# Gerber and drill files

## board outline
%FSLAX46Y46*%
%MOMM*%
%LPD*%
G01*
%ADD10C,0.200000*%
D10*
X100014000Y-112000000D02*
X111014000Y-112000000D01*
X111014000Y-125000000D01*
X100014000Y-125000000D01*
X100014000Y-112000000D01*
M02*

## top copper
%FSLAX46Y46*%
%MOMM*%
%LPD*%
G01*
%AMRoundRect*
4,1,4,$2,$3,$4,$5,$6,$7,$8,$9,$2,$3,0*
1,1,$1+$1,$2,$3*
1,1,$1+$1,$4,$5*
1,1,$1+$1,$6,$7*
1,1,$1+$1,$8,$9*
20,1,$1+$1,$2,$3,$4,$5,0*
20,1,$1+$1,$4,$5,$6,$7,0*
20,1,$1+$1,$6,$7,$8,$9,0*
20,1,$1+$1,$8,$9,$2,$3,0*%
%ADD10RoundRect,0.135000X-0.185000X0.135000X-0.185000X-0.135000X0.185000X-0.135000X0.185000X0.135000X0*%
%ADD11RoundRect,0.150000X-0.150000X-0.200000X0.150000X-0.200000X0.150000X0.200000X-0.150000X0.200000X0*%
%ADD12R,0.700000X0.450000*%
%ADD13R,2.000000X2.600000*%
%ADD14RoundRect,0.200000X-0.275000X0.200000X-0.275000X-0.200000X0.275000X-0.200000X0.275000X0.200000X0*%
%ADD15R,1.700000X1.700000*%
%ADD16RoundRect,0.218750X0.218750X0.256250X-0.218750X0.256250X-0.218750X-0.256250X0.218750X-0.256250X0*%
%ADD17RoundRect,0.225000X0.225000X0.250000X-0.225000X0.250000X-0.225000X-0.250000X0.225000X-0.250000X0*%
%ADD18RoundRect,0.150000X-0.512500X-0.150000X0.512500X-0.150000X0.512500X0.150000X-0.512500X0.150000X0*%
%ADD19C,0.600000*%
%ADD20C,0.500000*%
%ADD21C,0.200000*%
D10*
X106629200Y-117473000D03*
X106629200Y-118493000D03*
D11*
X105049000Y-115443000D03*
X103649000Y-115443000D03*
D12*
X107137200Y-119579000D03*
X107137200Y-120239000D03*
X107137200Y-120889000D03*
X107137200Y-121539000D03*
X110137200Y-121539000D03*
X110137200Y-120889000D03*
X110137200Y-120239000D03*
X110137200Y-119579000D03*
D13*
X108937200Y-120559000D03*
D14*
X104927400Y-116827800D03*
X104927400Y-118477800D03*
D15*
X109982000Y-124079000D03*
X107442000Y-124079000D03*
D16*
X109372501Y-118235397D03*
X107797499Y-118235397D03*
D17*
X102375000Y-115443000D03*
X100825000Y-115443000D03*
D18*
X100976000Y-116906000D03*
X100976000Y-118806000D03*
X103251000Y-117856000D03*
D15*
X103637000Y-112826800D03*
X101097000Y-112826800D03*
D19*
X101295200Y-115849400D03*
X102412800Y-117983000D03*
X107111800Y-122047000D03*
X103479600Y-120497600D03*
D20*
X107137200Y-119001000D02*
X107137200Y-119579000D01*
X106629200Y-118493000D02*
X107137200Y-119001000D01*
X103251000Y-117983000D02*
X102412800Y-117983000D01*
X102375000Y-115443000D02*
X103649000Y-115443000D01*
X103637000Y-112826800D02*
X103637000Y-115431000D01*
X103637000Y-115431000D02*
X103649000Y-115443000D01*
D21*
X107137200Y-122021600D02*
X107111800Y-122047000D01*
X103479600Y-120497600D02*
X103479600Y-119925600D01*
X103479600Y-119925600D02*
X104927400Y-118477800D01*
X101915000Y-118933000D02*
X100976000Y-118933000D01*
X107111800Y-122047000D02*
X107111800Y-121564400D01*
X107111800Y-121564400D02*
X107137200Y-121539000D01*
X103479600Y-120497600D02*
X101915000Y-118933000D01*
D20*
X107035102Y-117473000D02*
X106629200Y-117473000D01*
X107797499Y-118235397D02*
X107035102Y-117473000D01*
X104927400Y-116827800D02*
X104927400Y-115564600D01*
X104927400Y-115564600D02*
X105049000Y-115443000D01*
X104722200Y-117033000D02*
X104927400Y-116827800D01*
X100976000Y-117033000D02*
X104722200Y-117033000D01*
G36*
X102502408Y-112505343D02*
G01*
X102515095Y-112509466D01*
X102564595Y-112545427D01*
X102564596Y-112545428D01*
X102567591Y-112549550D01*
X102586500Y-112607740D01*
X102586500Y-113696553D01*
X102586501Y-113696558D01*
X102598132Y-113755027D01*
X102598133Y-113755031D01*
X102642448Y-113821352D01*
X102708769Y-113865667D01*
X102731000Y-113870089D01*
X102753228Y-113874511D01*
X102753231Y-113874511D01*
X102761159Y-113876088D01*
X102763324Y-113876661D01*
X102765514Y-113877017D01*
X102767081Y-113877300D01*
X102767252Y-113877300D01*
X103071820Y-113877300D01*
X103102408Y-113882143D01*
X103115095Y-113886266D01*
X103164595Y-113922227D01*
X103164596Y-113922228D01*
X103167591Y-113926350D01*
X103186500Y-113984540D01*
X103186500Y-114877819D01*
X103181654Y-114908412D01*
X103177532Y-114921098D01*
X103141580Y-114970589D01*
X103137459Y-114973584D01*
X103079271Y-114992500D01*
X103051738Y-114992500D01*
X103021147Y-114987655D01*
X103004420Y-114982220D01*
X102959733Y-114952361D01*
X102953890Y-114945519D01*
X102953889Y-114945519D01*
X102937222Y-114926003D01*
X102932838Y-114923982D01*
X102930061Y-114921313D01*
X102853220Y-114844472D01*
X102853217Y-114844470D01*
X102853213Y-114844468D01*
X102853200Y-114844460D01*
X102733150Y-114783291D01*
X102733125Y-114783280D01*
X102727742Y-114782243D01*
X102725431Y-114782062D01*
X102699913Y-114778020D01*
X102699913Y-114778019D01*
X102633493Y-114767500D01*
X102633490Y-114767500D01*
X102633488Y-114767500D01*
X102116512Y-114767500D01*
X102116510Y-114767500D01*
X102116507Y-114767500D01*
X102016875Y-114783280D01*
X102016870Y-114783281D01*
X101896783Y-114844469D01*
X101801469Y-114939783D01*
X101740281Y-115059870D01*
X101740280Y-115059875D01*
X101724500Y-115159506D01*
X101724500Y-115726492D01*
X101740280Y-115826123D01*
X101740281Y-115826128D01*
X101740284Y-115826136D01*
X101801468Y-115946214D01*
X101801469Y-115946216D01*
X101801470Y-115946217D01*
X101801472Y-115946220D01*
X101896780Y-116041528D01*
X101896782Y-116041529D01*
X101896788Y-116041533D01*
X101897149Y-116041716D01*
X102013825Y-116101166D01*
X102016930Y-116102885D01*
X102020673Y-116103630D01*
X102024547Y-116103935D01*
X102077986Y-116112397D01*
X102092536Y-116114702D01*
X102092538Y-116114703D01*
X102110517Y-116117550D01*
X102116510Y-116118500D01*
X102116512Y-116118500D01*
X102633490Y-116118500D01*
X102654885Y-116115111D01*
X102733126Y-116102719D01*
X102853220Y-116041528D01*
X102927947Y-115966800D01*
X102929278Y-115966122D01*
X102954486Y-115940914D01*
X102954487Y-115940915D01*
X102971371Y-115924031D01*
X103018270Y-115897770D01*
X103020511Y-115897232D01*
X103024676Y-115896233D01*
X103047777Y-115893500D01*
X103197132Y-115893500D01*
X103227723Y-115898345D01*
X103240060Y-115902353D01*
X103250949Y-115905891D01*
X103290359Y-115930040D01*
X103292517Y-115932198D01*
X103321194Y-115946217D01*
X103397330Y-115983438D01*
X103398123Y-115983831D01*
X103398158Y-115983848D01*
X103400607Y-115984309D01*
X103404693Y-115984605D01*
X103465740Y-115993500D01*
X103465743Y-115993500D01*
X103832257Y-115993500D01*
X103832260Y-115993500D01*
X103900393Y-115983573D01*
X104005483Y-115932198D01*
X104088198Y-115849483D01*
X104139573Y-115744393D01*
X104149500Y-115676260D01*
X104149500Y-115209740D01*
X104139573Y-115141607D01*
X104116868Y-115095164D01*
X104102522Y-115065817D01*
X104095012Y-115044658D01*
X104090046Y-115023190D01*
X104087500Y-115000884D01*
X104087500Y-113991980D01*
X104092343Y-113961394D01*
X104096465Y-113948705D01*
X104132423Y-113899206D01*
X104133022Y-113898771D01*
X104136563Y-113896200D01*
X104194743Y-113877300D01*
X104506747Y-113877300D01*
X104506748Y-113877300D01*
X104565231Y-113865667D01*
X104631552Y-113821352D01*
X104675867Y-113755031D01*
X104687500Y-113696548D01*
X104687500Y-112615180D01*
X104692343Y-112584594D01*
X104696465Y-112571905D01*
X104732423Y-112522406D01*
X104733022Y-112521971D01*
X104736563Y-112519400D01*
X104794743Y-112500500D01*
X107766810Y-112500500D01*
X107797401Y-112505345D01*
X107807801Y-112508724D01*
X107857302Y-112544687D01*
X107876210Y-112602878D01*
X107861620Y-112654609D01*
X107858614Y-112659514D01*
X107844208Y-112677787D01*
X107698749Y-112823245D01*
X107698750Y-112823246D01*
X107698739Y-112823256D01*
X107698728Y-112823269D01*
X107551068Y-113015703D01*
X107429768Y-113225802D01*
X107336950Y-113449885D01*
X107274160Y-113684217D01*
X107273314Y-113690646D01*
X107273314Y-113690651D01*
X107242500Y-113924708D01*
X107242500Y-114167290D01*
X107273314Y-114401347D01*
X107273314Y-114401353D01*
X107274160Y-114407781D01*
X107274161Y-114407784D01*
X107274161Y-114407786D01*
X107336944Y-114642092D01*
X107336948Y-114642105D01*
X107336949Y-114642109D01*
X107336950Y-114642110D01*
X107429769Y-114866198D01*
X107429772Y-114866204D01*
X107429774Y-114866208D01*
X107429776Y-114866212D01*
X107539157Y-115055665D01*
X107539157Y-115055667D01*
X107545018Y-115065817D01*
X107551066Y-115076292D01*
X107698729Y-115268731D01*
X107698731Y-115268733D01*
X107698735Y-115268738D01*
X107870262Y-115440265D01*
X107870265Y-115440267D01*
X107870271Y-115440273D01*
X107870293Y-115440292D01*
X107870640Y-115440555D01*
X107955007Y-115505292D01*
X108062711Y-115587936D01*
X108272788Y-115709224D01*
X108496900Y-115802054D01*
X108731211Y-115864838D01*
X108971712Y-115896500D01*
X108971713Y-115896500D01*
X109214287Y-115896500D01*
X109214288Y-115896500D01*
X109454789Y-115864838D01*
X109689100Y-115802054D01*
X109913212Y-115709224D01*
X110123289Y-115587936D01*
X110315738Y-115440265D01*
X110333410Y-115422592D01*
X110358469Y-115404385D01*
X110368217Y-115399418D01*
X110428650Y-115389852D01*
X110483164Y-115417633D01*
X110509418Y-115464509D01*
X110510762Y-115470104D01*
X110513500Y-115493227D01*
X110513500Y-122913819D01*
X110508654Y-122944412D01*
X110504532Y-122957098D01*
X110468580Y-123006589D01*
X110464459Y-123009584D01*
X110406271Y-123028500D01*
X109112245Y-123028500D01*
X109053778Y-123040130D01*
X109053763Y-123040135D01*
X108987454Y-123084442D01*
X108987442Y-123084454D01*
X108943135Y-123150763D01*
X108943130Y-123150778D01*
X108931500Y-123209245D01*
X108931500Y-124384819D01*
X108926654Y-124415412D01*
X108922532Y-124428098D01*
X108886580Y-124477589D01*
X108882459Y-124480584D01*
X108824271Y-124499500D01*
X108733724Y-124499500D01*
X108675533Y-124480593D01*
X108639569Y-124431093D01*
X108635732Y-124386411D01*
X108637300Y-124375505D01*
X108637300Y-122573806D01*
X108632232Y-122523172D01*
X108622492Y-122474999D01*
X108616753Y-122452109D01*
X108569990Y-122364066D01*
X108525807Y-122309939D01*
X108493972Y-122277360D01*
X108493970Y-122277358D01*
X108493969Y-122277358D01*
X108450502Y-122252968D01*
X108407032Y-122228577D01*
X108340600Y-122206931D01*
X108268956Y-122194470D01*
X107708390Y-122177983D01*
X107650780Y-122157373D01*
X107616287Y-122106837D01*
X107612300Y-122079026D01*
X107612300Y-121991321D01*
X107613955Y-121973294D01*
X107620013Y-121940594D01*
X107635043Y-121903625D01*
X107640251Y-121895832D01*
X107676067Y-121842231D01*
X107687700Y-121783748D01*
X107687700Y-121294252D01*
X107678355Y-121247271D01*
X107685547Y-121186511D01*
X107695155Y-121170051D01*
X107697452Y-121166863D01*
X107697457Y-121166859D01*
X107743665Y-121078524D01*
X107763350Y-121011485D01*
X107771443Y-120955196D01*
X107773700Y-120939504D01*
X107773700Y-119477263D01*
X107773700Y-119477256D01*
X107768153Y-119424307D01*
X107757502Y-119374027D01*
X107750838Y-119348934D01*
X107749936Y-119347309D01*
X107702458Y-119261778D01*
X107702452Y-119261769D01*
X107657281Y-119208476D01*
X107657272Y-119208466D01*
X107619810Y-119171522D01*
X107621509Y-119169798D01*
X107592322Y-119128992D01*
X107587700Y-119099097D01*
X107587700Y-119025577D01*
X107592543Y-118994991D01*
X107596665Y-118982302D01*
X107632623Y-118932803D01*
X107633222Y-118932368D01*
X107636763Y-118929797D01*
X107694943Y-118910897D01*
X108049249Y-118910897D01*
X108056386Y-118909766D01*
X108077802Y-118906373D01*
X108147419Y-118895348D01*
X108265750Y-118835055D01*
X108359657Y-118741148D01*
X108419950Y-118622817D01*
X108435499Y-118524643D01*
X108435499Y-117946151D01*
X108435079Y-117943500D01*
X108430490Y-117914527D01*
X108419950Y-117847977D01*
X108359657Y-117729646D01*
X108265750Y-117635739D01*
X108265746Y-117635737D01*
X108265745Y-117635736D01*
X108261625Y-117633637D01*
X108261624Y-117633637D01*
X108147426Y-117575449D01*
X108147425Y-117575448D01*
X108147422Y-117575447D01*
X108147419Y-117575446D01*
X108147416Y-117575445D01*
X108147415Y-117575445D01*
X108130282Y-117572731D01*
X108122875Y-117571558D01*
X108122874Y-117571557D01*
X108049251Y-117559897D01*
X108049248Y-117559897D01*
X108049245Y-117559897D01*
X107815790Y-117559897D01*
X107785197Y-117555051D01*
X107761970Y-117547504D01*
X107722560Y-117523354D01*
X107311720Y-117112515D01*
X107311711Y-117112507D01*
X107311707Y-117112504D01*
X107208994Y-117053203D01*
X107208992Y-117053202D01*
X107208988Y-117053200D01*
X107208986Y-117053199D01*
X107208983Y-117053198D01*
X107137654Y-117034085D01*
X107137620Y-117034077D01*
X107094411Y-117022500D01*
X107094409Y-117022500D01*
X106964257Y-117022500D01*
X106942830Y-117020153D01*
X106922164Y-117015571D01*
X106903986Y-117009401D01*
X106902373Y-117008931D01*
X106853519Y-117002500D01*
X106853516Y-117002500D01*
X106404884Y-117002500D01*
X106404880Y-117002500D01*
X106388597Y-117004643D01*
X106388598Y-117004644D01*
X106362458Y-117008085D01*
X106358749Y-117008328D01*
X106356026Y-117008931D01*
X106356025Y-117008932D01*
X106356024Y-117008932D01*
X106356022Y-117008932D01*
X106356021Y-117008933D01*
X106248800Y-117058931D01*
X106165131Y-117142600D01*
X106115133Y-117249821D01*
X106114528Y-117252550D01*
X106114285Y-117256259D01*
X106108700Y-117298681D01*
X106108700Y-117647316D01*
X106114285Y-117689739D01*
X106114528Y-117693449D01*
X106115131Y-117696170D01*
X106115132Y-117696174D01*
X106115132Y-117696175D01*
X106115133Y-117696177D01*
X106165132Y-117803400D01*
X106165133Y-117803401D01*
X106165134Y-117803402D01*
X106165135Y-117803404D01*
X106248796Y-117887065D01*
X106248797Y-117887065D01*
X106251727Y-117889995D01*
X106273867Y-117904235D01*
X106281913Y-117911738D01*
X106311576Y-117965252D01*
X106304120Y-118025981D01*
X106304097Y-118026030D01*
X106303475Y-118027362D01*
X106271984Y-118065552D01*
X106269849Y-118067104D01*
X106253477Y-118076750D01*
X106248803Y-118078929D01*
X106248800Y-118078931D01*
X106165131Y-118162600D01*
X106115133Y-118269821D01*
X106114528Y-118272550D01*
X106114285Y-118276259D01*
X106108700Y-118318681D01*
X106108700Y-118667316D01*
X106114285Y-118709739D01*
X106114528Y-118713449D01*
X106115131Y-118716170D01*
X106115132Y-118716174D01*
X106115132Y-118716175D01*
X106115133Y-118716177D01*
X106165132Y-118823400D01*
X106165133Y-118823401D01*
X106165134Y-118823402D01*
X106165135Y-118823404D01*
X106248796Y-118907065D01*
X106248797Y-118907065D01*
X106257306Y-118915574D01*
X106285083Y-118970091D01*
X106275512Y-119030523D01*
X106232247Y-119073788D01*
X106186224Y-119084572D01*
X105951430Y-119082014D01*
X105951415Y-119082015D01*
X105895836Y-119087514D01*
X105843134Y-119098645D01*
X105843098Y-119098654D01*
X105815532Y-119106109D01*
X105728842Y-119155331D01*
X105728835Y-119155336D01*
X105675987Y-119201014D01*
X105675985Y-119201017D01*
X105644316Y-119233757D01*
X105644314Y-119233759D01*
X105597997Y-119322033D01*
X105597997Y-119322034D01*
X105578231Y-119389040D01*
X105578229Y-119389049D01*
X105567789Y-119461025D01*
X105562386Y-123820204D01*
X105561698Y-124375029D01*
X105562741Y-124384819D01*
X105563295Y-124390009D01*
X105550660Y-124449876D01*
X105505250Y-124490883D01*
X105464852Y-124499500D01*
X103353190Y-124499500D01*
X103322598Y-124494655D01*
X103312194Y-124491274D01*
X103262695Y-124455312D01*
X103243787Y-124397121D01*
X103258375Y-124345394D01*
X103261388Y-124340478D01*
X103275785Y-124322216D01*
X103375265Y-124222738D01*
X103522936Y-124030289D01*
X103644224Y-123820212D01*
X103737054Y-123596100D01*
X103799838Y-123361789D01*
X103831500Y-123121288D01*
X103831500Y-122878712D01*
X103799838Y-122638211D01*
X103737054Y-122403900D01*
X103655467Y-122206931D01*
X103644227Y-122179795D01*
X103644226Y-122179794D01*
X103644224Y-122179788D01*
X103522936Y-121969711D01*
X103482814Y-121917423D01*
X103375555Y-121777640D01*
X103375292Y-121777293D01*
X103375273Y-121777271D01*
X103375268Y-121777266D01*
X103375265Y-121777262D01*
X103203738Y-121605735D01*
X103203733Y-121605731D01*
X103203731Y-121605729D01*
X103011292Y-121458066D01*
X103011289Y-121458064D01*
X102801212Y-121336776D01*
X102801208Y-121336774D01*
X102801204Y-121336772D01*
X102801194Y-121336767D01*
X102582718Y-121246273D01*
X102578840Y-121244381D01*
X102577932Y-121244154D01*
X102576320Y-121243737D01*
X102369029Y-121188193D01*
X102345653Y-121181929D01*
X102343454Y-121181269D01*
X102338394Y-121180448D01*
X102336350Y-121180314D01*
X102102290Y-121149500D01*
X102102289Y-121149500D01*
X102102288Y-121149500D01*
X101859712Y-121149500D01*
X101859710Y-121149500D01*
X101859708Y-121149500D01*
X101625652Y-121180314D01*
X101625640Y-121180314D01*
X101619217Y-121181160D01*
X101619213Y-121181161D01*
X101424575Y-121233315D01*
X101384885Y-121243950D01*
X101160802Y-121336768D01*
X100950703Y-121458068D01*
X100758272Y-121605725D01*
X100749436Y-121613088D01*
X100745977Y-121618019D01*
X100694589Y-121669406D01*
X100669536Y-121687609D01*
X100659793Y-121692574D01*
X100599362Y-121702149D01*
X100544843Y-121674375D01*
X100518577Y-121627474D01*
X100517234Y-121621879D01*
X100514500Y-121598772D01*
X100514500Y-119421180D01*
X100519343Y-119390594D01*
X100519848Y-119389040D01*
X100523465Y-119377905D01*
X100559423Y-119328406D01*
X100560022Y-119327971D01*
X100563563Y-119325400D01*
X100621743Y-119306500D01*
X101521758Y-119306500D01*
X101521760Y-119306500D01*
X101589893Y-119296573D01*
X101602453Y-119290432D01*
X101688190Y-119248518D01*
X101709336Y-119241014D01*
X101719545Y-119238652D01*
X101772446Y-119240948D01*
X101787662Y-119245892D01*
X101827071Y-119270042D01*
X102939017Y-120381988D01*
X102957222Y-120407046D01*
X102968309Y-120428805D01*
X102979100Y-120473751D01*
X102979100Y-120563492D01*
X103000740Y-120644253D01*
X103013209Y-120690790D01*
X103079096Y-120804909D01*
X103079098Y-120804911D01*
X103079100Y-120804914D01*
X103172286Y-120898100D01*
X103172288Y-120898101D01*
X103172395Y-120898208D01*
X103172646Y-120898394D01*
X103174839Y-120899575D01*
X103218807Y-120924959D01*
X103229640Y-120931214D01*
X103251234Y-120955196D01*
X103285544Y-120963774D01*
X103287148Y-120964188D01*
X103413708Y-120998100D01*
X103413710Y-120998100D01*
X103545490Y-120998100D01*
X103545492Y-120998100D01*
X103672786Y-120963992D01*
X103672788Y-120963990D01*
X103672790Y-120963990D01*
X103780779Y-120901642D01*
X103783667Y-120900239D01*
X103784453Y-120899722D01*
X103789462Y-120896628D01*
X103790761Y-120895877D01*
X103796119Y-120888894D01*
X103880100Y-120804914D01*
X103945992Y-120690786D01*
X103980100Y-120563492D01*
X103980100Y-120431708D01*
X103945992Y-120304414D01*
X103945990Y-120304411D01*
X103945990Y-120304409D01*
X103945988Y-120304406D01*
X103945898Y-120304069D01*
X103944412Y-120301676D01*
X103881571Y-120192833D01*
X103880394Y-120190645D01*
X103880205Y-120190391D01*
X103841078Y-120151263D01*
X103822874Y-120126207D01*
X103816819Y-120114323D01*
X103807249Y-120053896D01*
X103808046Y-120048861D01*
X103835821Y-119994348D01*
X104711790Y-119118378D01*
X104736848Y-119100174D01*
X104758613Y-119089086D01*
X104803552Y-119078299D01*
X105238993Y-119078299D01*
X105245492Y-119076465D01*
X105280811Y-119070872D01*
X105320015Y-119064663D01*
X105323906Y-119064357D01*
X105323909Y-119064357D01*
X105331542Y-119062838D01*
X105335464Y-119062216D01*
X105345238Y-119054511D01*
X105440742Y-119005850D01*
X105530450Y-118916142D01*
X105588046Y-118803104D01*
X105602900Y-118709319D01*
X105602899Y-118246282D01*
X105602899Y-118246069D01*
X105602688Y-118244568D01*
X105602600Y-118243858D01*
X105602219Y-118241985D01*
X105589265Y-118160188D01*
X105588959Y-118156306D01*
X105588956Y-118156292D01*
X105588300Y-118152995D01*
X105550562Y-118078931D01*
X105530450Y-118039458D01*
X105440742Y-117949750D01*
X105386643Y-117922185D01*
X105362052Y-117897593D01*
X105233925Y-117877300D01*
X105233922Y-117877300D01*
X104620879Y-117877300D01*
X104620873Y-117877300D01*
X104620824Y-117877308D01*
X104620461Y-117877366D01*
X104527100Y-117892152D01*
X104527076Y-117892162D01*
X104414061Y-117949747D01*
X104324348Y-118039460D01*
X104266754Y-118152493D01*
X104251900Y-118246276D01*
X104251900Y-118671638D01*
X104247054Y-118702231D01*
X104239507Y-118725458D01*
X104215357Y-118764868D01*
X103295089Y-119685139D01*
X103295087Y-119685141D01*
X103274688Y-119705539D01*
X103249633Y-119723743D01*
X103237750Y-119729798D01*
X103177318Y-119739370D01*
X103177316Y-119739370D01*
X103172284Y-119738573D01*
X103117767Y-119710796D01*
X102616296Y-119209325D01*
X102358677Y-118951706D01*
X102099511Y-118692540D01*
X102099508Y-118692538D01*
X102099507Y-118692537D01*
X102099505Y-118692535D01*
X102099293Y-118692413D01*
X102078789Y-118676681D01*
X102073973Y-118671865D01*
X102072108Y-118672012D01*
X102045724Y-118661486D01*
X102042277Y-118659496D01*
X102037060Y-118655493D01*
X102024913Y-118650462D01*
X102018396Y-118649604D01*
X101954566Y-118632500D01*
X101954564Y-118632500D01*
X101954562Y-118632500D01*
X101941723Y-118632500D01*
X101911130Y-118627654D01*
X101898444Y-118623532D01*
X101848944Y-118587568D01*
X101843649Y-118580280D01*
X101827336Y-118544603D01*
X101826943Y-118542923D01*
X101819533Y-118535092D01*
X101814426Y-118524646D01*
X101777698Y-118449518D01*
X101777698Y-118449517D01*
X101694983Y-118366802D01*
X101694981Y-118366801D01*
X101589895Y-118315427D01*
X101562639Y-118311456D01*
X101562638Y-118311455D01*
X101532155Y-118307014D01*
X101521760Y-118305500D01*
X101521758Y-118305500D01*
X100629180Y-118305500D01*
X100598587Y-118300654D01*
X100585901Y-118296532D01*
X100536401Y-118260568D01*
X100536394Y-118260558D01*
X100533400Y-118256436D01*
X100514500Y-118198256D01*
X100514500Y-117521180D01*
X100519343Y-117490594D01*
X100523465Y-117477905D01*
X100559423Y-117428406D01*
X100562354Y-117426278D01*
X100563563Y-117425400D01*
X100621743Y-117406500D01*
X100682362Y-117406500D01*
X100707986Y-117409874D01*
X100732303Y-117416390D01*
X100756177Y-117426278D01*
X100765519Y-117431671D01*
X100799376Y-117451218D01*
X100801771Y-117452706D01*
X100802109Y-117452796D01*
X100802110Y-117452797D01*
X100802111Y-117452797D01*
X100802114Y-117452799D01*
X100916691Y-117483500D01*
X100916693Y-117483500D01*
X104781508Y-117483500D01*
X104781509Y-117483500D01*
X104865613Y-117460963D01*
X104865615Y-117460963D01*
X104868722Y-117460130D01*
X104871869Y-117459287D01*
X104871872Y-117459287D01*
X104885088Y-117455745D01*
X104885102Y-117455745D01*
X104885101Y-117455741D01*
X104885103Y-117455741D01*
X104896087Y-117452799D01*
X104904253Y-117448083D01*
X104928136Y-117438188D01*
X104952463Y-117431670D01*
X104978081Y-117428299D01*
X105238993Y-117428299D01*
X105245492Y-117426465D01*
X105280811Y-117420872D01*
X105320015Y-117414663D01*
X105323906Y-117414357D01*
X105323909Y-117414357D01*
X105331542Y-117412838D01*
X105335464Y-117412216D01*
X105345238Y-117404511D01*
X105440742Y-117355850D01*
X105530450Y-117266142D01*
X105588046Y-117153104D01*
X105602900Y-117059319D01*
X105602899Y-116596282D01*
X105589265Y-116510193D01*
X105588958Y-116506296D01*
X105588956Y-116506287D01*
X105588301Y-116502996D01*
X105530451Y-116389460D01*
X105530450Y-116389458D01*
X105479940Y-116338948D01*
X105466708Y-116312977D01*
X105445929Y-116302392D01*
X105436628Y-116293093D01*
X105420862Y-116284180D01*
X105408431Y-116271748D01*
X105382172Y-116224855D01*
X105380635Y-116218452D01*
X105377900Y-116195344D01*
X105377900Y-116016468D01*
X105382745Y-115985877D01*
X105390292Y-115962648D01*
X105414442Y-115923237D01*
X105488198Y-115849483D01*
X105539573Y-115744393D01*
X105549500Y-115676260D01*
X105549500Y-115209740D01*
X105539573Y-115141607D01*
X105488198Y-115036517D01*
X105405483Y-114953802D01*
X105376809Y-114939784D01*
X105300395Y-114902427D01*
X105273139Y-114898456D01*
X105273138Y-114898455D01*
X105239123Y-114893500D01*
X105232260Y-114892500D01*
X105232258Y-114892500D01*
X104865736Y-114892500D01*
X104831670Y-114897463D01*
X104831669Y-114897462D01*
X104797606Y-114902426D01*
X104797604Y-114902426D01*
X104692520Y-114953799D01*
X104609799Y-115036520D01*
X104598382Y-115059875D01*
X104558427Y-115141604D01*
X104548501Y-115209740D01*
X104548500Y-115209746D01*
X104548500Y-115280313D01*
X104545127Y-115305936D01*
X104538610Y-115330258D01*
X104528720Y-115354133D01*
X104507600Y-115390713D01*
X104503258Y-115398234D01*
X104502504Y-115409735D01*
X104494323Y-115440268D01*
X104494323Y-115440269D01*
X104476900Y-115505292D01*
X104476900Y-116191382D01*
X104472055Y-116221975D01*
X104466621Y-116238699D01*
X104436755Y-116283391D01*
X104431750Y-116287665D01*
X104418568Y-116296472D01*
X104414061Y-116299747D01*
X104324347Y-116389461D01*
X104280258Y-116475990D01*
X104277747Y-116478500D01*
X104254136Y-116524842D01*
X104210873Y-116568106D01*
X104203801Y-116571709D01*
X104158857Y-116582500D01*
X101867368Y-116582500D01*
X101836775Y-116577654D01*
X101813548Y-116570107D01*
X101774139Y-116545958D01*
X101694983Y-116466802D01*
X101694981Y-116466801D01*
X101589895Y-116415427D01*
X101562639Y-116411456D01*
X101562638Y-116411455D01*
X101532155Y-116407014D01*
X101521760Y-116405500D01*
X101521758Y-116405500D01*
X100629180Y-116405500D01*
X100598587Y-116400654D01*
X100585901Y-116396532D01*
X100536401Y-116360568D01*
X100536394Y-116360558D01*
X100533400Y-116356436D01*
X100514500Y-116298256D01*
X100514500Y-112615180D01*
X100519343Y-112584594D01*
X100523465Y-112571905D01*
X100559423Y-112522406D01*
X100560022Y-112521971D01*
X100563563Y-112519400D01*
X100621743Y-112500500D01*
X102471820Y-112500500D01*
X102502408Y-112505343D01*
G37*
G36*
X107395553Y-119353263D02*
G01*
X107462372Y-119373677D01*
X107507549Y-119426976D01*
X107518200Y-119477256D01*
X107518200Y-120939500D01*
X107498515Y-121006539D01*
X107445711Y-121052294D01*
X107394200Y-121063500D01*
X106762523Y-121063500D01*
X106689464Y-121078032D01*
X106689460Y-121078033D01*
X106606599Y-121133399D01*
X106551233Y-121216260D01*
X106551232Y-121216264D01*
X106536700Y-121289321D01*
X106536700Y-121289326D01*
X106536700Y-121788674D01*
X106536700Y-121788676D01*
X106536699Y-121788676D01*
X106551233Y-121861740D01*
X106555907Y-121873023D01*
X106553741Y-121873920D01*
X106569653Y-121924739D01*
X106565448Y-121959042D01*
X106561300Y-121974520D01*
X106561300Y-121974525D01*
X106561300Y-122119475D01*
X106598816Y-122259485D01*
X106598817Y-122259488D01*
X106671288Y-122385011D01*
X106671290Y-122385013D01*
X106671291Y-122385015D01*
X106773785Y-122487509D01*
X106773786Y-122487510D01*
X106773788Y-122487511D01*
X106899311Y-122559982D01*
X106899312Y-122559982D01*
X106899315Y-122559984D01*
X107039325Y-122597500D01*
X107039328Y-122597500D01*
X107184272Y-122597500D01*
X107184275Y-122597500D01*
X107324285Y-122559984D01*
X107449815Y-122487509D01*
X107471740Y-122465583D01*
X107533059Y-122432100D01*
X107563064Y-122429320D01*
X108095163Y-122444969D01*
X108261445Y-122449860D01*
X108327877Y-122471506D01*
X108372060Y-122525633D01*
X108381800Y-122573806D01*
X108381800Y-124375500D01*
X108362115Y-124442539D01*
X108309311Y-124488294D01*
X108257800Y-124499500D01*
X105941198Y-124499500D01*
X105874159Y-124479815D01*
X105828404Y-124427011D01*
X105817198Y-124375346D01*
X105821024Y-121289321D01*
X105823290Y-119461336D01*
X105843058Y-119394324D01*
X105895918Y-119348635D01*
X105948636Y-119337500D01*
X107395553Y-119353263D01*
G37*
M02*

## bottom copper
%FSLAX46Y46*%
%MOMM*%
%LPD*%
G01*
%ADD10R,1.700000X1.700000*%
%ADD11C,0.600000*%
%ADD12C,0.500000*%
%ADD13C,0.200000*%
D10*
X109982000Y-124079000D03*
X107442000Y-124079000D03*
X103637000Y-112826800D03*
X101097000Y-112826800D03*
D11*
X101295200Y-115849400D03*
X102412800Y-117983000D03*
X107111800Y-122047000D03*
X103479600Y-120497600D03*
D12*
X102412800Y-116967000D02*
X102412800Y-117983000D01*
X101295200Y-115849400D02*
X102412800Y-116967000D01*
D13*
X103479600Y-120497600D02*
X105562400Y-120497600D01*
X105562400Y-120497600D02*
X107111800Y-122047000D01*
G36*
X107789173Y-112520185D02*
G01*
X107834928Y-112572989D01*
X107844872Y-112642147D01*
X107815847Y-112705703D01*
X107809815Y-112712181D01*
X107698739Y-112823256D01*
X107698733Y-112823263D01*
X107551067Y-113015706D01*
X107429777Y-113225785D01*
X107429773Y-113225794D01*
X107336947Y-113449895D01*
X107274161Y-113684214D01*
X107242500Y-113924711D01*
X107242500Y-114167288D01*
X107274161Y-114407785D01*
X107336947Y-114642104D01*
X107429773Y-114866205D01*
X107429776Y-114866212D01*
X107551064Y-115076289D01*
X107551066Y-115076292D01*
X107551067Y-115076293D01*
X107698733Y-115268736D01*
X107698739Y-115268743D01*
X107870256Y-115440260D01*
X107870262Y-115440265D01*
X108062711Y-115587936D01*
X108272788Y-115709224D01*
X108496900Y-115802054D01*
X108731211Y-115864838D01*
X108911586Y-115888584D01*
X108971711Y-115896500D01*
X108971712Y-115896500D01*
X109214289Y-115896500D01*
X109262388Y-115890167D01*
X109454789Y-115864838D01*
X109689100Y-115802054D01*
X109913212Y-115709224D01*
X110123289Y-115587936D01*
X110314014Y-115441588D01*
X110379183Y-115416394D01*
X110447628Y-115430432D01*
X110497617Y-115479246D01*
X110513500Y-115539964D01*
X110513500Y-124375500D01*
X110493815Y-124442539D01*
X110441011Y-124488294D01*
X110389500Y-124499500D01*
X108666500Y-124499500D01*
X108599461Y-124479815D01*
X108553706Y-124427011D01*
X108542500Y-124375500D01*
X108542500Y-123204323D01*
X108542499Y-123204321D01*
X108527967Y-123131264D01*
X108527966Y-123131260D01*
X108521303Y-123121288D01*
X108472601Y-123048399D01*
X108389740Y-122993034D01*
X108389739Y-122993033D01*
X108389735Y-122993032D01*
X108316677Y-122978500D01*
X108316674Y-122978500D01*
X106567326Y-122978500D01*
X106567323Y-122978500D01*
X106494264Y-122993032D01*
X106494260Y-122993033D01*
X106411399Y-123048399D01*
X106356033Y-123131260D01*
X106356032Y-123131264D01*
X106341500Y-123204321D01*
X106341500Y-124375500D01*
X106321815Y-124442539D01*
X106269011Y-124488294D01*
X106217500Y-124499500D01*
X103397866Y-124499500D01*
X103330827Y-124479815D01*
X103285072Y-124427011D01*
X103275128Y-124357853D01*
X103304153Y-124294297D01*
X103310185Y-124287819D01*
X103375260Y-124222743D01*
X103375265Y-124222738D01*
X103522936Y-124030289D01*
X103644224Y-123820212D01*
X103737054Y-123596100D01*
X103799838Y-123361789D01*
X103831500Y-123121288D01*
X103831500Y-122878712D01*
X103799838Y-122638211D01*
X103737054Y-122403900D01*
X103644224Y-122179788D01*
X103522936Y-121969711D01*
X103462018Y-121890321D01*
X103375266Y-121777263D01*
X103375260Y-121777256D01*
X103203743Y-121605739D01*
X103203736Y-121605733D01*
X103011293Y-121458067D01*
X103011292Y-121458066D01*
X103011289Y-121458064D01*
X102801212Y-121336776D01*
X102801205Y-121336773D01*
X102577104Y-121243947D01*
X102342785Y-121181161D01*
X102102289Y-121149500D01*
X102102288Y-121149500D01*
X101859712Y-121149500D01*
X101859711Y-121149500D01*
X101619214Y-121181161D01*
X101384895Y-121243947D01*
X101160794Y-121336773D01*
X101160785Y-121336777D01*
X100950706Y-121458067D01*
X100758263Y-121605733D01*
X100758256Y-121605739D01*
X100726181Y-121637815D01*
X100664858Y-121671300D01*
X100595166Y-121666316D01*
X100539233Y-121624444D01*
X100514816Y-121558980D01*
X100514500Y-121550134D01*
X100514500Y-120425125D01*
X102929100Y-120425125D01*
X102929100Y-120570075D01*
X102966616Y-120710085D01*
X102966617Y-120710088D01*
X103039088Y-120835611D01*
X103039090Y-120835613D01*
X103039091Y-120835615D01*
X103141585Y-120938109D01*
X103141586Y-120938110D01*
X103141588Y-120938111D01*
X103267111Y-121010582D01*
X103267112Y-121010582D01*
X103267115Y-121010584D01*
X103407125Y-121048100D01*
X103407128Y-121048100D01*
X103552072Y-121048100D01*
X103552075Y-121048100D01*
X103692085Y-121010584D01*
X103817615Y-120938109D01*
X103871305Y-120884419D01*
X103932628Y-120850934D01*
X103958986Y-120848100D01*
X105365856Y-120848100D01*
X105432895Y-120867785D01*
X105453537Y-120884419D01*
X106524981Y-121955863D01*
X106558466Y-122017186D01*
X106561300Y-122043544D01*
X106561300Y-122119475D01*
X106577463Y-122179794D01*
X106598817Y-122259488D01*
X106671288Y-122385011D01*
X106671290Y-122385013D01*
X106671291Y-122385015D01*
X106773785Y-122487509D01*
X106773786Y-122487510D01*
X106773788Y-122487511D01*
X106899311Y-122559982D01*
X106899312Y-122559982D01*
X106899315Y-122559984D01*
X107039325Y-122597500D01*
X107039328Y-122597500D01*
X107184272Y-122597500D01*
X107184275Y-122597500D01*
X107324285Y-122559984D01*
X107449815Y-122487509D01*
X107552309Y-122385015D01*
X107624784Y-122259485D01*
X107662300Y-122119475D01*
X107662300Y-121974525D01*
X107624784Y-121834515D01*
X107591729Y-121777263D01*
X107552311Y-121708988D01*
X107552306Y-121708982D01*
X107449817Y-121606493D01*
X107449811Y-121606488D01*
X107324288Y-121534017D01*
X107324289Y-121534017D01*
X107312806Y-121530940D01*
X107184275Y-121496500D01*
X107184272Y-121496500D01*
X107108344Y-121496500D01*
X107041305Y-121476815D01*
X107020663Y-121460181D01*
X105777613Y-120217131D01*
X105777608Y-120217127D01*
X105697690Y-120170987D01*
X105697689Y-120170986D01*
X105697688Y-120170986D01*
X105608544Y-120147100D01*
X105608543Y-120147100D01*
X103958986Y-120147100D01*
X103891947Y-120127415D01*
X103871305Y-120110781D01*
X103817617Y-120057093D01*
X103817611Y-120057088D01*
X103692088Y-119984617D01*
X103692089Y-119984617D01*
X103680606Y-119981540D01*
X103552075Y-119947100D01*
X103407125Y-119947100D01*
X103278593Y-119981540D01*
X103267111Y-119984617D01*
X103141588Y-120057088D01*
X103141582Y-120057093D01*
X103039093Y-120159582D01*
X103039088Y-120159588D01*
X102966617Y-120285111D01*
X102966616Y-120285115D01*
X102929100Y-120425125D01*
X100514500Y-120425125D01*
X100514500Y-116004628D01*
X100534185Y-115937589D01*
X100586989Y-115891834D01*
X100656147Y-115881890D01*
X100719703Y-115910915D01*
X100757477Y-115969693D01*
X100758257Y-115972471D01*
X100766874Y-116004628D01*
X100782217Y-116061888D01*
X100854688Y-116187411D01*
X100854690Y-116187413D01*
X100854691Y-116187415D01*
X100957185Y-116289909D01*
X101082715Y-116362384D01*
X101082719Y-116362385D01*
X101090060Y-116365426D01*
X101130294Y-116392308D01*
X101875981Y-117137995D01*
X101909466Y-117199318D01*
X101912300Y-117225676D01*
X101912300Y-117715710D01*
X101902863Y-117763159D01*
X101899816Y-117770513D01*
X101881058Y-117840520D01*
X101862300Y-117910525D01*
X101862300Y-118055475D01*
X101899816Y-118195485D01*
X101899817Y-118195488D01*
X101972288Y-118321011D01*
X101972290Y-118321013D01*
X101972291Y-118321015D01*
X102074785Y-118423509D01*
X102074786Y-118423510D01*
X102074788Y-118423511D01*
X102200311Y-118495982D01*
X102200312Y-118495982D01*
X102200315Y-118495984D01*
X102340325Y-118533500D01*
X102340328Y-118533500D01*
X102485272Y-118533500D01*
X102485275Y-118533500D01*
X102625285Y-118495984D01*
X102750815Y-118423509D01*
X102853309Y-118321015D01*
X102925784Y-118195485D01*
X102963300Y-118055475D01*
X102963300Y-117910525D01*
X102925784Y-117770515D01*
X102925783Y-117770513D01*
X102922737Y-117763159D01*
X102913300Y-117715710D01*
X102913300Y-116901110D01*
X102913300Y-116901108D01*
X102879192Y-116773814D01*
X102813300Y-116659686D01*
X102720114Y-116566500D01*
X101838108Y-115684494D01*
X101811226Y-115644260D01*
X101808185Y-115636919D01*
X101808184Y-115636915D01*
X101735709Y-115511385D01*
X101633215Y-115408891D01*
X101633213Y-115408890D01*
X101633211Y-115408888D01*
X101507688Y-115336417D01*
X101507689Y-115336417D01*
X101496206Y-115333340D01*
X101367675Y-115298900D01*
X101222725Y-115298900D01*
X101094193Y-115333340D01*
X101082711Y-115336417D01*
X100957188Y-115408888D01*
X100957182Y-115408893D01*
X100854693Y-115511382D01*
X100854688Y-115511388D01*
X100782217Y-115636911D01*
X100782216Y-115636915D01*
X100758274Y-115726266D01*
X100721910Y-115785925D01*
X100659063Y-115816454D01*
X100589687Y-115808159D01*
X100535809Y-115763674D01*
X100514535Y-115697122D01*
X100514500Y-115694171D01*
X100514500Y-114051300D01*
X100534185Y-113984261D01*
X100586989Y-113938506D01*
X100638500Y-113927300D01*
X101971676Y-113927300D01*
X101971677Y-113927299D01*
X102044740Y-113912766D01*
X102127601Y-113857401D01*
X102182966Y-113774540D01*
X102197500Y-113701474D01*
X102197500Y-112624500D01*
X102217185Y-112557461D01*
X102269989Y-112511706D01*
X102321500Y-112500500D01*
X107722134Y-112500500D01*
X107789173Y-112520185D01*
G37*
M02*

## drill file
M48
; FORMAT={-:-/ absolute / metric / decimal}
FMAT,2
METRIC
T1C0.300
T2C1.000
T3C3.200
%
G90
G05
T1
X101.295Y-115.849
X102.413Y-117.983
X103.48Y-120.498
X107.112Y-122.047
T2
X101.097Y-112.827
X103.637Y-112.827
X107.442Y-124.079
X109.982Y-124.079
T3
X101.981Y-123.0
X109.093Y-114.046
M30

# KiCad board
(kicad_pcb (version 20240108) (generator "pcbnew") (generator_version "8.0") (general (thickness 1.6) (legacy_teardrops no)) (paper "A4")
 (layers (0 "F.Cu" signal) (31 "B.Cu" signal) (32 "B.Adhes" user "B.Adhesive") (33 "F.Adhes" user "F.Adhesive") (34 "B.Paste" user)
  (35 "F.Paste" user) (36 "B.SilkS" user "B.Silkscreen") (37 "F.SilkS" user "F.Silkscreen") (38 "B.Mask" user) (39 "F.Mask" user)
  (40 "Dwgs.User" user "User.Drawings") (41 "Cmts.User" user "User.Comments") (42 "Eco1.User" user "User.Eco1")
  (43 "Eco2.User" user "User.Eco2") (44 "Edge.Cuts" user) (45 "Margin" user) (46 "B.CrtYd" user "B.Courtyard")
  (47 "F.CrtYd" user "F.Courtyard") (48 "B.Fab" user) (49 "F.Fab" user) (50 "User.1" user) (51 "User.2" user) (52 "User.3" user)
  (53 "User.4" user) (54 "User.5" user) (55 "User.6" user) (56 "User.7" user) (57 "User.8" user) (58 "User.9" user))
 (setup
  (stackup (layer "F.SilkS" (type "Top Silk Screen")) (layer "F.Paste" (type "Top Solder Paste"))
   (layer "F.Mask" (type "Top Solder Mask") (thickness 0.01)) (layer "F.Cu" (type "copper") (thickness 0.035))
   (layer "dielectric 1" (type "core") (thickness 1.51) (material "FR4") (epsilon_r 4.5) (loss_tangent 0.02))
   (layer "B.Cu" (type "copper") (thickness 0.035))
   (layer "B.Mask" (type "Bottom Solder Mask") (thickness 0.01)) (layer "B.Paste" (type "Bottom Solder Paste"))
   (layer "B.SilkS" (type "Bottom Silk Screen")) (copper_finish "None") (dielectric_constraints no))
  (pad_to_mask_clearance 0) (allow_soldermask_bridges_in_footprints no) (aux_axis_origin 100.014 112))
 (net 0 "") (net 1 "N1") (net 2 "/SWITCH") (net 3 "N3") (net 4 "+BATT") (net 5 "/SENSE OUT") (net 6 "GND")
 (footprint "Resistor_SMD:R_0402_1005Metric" (layer "F.Cu") (at 106.6292 117.983 -90)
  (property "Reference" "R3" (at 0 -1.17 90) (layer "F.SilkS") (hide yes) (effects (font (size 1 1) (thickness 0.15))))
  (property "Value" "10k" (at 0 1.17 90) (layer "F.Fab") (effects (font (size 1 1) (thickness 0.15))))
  (pad "1" smd roundrect (at -0.51 0 270) (size 0.54 0.64) (layers "F.Cu" "F.Paste" "F.Mask") (roundrect_rratio 0.25) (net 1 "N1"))
  (pad "2" smd roundrect (at 0.51 0 270) (size 0.54 0.64) (layers "F.Cu" "F.Paste" "F.Mask") (roundrect_rratio 0.25) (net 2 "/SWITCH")))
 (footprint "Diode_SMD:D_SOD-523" (layer "F.Cu") (at 104.349 115.443 180)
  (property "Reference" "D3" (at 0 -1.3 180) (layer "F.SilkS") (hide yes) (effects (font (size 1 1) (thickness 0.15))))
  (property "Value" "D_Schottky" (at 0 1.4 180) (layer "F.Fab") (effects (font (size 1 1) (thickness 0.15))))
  (pad "1" smd roundrect (at -0.7 0) (size 0.6 0.7) (layers "F.Cu" "F.Paste" "F.Mask") (roundrect_rratio 0.25) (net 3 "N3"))
  (pad "2" smd roundrect (at 0.7 0) (size 0.6 0.7) (layers "F.Cu" "F.Paste" "F.Mask") (roundrect_rratio 0.25) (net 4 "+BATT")))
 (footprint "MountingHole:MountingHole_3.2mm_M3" (layer "F.Cu") (at 101.981 123)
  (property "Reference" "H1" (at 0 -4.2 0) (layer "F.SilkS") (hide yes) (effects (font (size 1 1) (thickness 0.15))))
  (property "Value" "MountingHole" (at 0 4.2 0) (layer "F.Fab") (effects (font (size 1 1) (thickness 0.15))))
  (pad "" np_thru_hole circle (at 0 0) (size 3.2 3.2) (drill 3.2) (layers "*.Cu" "*.Mask")))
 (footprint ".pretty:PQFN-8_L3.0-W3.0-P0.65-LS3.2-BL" (layer "F.Cu") (at 108.6372 120.559 -90)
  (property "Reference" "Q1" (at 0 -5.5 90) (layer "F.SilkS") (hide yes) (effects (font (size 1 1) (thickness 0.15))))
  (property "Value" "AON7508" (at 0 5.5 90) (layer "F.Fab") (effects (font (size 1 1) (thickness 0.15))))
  (pad "1" smd rect (at -0.98 1.5 270) (size 0.45 0.7) (layers "F.Cu" "F.Paste" "F.Mask") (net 2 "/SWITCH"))
  (pad "2" smd rect (at -0.32 1.5 270) (size 0.45 0.7) (layers "F.Cu" "F.Paste" "F.Mask") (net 2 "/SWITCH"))
  (pad "3" smd rect (at 0.33 1.5 270) (size 0.45 0.7) (layers "F.Cu" "F.Paste" "F.Mask") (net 2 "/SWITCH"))
  (pad "4" smd rect (at 0.98 1.5 270) (size 0.45 0.7) (layers "F.Cu" "F.Paste" "F.Mask") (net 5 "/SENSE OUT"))
  (pad "5" smd rect (at 0.98 -1.5 270) (size 0.45 0.7) (layers "F.Cu" "F.Paste" "F.Mask") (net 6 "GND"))
  (pad "6" smd rect (at 0.33 -1.5 270) (size 0.45 0.7) (layers "F.Cu" "F.Paste" "F.Mask") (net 6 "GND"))
  (pad "7" smd rect (at -0.32 -1.5 270) (size 0.45 0.7) (layers "F.Cu" "F.Paste" "F.Mask") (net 6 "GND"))
  (pad "8" smd rect (at -0.98 -1.5 270) (size 0.45 0.7) (layers "F.Cu" "F.Paste" "F.Mask") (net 6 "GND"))
  (pad "8" smd rect (at 0 -0.3 270) (size 2.6 2) (layers "F.Cu" "F.Paste" "F.Mask") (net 6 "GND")))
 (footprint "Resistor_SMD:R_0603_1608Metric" (layer "F.Cu") (at 104.9274 117.6528 -90)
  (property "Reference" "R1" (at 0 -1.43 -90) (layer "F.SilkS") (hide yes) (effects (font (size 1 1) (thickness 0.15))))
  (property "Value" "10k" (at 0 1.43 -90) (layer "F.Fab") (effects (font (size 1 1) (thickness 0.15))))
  (pad "1" smd roundrect (at -0.825 0 270) (size 0.8 0.95) (layers "F.Cu" "F.Paste" "F.Mask") (roundrect_rratio 0.25) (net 3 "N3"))
  (pad "2" smd roundrect (at 0.825 0 270) (size 0.8 0.95) (layers "F.Cu" "F.Paste" "F.Mask") (roundrect_rratio 0.25) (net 5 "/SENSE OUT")))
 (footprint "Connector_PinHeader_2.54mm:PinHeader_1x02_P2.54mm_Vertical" (layer "F.Cu") (at 109.982 124.079 -90)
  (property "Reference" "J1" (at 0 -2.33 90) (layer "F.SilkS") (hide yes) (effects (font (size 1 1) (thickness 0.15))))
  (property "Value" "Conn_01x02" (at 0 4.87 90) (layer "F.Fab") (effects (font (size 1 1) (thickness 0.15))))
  (pad "1" thru_hole rect (at 0 0 270) (size 1.7 1.7) (drill 1) (layers "*.Cu" "*.Mask") (remove_unused_layers no) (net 4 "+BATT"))
  (pad "2" thru_hole rect (at 0 2.54 270) (size 1.7 1.7) (drill 1) (layers "*.Cu" "*.Mask") (remove_unused_layers no) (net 2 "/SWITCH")))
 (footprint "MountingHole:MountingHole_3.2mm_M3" (layer "F.Cu") (at 109.093 114.046)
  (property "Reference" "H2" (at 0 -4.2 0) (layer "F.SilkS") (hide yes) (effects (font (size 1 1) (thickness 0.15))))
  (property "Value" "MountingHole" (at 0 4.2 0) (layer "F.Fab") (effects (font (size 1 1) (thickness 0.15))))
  (pad "" np_thru_hole circle (at 0 0) (size 3.2 3.2) (drill 3.2) (layers "*.Cu" "*.Mask")))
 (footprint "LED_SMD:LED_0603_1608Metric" (layer "F.Cu") (at 108.585 118.235397 180)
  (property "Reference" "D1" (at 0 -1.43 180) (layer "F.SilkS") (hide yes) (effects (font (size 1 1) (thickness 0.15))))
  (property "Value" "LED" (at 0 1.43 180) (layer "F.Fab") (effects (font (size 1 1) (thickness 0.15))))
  (pad "1" smd roundrect (at -0.787501 0 180) (size 0.875 0.95) (layers "F.Cu" "F.Paste" "F.Mask") (roundrect_rratio 0.25) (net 6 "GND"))
  (pad "2" smd roundrect (at 0.787501 0 180) (size 0.875 0.95) (layers "F.Cu" "F.Paste" "F.Mask") (roundrect_rratio 0.25) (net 1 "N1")))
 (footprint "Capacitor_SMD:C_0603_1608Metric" (layer "F.Cu") (at 101.6 115.443 180)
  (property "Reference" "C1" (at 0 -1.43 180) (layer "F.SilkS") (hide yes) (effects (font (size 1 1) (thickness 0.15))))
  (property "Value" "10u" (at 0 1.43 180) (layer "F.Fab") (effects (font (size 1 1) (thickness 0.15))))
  (pad "1" smd roundrect (at -0.775 0 180) (size 0.9 0.95) (layers "F.Cu" "F.Paste" "F.Mask") (roundrect_rratio 0.25) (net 4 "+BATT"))
  (pad "2" smd roundrect (at 0.775 0 180) (size 0.9 0.95) (layers "F.Cu" "F.Paste" "F.Mask") (roundrect_rratio 0.25) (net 6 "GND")))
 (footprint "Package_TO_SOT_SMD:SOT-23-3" (layer "F.Cu") (at 102.1135 117.856)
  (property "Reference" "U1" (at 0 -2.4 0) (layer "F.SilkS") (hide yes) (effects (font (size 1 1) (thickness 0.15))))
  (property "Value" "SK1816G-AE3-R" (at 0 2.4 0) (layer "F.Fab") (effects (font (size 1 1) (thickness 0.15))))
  (pad "1" smd roundrect (at -1.1375 -0.95) (size 1.325 0.6) (layers "F.Cu" "F.Paste" "F.Mask") (roundrect_rratio 0.25) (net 3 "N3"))
  (pad "2" smd roundrect (at -1.1375 0.95) (size 1.325 0.6) (layers "F.Cu" "F.Paste" "F.Mask") (roundrect_rratio 0.25) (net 5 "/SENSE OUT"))
  (pad "3" smd roundrect (at 1.1375 0) (size 1.325 0.6) (layers "F.Cu" "F.Paste" "F.Mask") (roundrect_rratio 0.25) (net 6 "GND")))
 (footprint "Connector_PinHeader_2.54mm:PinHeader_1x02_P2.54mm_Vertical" (layer "F.Cu") (at 103.637 112.8268 -90)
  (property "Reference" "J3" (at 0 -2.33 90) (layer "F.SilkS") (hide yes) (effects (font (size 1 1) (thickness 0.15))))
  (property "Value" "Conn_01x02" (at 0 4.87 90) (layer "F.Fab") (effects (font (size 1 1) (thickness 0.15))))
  (pad "1" thru_hole rect (at 0 0 270) (size 1.7 1.7) (drill 1) (layers "*.Cu" "*.Mask") (remove_unused_layers no) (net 4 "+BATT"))
  (pad "2" thru_hole rect (at 0 2.54 270) (size 1.7 1.7) (drill 1) (layers "*.Cu" "*.Mask") (remove_unused_layers no) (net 6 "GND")))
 (gr_rect (start 100.014 112) (end 111.014 125) (stroke (width 0.2) (type default)) (fill none) (layer "Edge.Cuts"))
 (segment (start 107.1372 119.001) (end 107.1372 119.579) (width 0.5) (layer "F.Cu") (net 2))
 (segment (start 106.6292 118.493) (end 107.1372 119.001) (width 0.5) (layer "F.Cu") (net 2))
 (segment (start 103.251 117.983) (end 102.4128 117.983) (width 0.5) (layer "F.Cu") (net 6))
 (via (at 101.2952 115.8494) (size 0.6) (drill 0.3) (layers "F.Cu" "B.Cu") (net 6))
 (via (at 102.4128 117.983) (size 0.6) (drill 0.3) (layers "F.Cu" "B.Cu") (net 6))
 (segment (start 102.4128 116.967) (end 102.4128 117.983) (width 0.5) (layer "B.Cu") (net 6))
 (segment (start 101.2952 115.8494) (end 102.4128 116.967) (width 0.5) (layer "B.Cu") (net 6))
 (segment (start 102.375 115.443) (end 103.649 115.443) (width 0.5) (layer "F.Cu") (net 4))
 (segment (start 103.637 112.8268) (end 103.637 115.431) (width 0.5) (layer "F.Cu") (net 4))
 (segment (start 103.637 115.431) (end 103.649 115.443) (width 0.5) (layer "F.Cu") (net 4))
 (segment (start 107.1372 122.0216) (end 107.1118 122.047) (width 0.2) (layer "F.Cu") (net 5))
 (segment (start 103.4796 120.4976) (end 103.4796 119.9256) (width 0.2) (layer "F.Cu") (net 5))
 (segment (start 103.4796 119.9256) (end 104.9274 118.4778) (width 0.2) (layer "F.Cu") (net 5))
 (segment (start 101.915 118.933) (end 100.976 118.933) (width 0.2) (layer "F.Cu") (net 5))
 (segment (start 107.1118 122.047) (end 107.1118 121.5644) (width 0.2) (layer "F.Cu") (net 5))
 (segment (start 107.1118 121.5644) (end 107.1372 121.539) (width 0.2) (layer "F.Cu") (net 5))
 (segment (start 103.4796 120.4976) (end 101.915 118.933) (width 0.2) (layer "F.Cu") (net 5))
 (via (at 107.1118 122.047) (size 0.6) (drill 0.3) (layers "F.Cu" "B.Cu") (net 5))
 (via (at 103.4796 120.4976) (size 0.6) (drill 0.3) (layers "F.Cu" "B.Cu") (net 5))
 (segment (start 103.4796 120.4976) (end 105.5624 120.4976) (width 0.2) (layer "B.Cu") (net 5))
 (segment (start 105.5624 120.4976) (end 107.1118 122.047) (width 0.2) (layer "B.Cu") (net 5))
 (segment (start 107.035102 117.473) (end 106.6292 117.473) (width 0.5) (layer "F.Cu") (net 1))
 (segment (start 107.797499 118.235397) (end 107.035102 117.473) (width 0.5) (layer "F.Cu") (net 1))
 (segment (start 104.9274 116.8278) (end 104.9274 115.5646) (width 0.5) (layer "F.Cu") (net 3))
 (segment (start 104.9274 115.5646) (end 105.049 115.443) (width 0.5) (layer "F.Cu") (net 3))
 (segment (start 104.7222 117.033) (end 104.9274 116.8278) (width 0.5) (layer "F.Cu") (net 3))
 (segment (start 100.976 117.033) (end 104.7222 117.033) (width 0.5) (layer "F.Cu") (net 3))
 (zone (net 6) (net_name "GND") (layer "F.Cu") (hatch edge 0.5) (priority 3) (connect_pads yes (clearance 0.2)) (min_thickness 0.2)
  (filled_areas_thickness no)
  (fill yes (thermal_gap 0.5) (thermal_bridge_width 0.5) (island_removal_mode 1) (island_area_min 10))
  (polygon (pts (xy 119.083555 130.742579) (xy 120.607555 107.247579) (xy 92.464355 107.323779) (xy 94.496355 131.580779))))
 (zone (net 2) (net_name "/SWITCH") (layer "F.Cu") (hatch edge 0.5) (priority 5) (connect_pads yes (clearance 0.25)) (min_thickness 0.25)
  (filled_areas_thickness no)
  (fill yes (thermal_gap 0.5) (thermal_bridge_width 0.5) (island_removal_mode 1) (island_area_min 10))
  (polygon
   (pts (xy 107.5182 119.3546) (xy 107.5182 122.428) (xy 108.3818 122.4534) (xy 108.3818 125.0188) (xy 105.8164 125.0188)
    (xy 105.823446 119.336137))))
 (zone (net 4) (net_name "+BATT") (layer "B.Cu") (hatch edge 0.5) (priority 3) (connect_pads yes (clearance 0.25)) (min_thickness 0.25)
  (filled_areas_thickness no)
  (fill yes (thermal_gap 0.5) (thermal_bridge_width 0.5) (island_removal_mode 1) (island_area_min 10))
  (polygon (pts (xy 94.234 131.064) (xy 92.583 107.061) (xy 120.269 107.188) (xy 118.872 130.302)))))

